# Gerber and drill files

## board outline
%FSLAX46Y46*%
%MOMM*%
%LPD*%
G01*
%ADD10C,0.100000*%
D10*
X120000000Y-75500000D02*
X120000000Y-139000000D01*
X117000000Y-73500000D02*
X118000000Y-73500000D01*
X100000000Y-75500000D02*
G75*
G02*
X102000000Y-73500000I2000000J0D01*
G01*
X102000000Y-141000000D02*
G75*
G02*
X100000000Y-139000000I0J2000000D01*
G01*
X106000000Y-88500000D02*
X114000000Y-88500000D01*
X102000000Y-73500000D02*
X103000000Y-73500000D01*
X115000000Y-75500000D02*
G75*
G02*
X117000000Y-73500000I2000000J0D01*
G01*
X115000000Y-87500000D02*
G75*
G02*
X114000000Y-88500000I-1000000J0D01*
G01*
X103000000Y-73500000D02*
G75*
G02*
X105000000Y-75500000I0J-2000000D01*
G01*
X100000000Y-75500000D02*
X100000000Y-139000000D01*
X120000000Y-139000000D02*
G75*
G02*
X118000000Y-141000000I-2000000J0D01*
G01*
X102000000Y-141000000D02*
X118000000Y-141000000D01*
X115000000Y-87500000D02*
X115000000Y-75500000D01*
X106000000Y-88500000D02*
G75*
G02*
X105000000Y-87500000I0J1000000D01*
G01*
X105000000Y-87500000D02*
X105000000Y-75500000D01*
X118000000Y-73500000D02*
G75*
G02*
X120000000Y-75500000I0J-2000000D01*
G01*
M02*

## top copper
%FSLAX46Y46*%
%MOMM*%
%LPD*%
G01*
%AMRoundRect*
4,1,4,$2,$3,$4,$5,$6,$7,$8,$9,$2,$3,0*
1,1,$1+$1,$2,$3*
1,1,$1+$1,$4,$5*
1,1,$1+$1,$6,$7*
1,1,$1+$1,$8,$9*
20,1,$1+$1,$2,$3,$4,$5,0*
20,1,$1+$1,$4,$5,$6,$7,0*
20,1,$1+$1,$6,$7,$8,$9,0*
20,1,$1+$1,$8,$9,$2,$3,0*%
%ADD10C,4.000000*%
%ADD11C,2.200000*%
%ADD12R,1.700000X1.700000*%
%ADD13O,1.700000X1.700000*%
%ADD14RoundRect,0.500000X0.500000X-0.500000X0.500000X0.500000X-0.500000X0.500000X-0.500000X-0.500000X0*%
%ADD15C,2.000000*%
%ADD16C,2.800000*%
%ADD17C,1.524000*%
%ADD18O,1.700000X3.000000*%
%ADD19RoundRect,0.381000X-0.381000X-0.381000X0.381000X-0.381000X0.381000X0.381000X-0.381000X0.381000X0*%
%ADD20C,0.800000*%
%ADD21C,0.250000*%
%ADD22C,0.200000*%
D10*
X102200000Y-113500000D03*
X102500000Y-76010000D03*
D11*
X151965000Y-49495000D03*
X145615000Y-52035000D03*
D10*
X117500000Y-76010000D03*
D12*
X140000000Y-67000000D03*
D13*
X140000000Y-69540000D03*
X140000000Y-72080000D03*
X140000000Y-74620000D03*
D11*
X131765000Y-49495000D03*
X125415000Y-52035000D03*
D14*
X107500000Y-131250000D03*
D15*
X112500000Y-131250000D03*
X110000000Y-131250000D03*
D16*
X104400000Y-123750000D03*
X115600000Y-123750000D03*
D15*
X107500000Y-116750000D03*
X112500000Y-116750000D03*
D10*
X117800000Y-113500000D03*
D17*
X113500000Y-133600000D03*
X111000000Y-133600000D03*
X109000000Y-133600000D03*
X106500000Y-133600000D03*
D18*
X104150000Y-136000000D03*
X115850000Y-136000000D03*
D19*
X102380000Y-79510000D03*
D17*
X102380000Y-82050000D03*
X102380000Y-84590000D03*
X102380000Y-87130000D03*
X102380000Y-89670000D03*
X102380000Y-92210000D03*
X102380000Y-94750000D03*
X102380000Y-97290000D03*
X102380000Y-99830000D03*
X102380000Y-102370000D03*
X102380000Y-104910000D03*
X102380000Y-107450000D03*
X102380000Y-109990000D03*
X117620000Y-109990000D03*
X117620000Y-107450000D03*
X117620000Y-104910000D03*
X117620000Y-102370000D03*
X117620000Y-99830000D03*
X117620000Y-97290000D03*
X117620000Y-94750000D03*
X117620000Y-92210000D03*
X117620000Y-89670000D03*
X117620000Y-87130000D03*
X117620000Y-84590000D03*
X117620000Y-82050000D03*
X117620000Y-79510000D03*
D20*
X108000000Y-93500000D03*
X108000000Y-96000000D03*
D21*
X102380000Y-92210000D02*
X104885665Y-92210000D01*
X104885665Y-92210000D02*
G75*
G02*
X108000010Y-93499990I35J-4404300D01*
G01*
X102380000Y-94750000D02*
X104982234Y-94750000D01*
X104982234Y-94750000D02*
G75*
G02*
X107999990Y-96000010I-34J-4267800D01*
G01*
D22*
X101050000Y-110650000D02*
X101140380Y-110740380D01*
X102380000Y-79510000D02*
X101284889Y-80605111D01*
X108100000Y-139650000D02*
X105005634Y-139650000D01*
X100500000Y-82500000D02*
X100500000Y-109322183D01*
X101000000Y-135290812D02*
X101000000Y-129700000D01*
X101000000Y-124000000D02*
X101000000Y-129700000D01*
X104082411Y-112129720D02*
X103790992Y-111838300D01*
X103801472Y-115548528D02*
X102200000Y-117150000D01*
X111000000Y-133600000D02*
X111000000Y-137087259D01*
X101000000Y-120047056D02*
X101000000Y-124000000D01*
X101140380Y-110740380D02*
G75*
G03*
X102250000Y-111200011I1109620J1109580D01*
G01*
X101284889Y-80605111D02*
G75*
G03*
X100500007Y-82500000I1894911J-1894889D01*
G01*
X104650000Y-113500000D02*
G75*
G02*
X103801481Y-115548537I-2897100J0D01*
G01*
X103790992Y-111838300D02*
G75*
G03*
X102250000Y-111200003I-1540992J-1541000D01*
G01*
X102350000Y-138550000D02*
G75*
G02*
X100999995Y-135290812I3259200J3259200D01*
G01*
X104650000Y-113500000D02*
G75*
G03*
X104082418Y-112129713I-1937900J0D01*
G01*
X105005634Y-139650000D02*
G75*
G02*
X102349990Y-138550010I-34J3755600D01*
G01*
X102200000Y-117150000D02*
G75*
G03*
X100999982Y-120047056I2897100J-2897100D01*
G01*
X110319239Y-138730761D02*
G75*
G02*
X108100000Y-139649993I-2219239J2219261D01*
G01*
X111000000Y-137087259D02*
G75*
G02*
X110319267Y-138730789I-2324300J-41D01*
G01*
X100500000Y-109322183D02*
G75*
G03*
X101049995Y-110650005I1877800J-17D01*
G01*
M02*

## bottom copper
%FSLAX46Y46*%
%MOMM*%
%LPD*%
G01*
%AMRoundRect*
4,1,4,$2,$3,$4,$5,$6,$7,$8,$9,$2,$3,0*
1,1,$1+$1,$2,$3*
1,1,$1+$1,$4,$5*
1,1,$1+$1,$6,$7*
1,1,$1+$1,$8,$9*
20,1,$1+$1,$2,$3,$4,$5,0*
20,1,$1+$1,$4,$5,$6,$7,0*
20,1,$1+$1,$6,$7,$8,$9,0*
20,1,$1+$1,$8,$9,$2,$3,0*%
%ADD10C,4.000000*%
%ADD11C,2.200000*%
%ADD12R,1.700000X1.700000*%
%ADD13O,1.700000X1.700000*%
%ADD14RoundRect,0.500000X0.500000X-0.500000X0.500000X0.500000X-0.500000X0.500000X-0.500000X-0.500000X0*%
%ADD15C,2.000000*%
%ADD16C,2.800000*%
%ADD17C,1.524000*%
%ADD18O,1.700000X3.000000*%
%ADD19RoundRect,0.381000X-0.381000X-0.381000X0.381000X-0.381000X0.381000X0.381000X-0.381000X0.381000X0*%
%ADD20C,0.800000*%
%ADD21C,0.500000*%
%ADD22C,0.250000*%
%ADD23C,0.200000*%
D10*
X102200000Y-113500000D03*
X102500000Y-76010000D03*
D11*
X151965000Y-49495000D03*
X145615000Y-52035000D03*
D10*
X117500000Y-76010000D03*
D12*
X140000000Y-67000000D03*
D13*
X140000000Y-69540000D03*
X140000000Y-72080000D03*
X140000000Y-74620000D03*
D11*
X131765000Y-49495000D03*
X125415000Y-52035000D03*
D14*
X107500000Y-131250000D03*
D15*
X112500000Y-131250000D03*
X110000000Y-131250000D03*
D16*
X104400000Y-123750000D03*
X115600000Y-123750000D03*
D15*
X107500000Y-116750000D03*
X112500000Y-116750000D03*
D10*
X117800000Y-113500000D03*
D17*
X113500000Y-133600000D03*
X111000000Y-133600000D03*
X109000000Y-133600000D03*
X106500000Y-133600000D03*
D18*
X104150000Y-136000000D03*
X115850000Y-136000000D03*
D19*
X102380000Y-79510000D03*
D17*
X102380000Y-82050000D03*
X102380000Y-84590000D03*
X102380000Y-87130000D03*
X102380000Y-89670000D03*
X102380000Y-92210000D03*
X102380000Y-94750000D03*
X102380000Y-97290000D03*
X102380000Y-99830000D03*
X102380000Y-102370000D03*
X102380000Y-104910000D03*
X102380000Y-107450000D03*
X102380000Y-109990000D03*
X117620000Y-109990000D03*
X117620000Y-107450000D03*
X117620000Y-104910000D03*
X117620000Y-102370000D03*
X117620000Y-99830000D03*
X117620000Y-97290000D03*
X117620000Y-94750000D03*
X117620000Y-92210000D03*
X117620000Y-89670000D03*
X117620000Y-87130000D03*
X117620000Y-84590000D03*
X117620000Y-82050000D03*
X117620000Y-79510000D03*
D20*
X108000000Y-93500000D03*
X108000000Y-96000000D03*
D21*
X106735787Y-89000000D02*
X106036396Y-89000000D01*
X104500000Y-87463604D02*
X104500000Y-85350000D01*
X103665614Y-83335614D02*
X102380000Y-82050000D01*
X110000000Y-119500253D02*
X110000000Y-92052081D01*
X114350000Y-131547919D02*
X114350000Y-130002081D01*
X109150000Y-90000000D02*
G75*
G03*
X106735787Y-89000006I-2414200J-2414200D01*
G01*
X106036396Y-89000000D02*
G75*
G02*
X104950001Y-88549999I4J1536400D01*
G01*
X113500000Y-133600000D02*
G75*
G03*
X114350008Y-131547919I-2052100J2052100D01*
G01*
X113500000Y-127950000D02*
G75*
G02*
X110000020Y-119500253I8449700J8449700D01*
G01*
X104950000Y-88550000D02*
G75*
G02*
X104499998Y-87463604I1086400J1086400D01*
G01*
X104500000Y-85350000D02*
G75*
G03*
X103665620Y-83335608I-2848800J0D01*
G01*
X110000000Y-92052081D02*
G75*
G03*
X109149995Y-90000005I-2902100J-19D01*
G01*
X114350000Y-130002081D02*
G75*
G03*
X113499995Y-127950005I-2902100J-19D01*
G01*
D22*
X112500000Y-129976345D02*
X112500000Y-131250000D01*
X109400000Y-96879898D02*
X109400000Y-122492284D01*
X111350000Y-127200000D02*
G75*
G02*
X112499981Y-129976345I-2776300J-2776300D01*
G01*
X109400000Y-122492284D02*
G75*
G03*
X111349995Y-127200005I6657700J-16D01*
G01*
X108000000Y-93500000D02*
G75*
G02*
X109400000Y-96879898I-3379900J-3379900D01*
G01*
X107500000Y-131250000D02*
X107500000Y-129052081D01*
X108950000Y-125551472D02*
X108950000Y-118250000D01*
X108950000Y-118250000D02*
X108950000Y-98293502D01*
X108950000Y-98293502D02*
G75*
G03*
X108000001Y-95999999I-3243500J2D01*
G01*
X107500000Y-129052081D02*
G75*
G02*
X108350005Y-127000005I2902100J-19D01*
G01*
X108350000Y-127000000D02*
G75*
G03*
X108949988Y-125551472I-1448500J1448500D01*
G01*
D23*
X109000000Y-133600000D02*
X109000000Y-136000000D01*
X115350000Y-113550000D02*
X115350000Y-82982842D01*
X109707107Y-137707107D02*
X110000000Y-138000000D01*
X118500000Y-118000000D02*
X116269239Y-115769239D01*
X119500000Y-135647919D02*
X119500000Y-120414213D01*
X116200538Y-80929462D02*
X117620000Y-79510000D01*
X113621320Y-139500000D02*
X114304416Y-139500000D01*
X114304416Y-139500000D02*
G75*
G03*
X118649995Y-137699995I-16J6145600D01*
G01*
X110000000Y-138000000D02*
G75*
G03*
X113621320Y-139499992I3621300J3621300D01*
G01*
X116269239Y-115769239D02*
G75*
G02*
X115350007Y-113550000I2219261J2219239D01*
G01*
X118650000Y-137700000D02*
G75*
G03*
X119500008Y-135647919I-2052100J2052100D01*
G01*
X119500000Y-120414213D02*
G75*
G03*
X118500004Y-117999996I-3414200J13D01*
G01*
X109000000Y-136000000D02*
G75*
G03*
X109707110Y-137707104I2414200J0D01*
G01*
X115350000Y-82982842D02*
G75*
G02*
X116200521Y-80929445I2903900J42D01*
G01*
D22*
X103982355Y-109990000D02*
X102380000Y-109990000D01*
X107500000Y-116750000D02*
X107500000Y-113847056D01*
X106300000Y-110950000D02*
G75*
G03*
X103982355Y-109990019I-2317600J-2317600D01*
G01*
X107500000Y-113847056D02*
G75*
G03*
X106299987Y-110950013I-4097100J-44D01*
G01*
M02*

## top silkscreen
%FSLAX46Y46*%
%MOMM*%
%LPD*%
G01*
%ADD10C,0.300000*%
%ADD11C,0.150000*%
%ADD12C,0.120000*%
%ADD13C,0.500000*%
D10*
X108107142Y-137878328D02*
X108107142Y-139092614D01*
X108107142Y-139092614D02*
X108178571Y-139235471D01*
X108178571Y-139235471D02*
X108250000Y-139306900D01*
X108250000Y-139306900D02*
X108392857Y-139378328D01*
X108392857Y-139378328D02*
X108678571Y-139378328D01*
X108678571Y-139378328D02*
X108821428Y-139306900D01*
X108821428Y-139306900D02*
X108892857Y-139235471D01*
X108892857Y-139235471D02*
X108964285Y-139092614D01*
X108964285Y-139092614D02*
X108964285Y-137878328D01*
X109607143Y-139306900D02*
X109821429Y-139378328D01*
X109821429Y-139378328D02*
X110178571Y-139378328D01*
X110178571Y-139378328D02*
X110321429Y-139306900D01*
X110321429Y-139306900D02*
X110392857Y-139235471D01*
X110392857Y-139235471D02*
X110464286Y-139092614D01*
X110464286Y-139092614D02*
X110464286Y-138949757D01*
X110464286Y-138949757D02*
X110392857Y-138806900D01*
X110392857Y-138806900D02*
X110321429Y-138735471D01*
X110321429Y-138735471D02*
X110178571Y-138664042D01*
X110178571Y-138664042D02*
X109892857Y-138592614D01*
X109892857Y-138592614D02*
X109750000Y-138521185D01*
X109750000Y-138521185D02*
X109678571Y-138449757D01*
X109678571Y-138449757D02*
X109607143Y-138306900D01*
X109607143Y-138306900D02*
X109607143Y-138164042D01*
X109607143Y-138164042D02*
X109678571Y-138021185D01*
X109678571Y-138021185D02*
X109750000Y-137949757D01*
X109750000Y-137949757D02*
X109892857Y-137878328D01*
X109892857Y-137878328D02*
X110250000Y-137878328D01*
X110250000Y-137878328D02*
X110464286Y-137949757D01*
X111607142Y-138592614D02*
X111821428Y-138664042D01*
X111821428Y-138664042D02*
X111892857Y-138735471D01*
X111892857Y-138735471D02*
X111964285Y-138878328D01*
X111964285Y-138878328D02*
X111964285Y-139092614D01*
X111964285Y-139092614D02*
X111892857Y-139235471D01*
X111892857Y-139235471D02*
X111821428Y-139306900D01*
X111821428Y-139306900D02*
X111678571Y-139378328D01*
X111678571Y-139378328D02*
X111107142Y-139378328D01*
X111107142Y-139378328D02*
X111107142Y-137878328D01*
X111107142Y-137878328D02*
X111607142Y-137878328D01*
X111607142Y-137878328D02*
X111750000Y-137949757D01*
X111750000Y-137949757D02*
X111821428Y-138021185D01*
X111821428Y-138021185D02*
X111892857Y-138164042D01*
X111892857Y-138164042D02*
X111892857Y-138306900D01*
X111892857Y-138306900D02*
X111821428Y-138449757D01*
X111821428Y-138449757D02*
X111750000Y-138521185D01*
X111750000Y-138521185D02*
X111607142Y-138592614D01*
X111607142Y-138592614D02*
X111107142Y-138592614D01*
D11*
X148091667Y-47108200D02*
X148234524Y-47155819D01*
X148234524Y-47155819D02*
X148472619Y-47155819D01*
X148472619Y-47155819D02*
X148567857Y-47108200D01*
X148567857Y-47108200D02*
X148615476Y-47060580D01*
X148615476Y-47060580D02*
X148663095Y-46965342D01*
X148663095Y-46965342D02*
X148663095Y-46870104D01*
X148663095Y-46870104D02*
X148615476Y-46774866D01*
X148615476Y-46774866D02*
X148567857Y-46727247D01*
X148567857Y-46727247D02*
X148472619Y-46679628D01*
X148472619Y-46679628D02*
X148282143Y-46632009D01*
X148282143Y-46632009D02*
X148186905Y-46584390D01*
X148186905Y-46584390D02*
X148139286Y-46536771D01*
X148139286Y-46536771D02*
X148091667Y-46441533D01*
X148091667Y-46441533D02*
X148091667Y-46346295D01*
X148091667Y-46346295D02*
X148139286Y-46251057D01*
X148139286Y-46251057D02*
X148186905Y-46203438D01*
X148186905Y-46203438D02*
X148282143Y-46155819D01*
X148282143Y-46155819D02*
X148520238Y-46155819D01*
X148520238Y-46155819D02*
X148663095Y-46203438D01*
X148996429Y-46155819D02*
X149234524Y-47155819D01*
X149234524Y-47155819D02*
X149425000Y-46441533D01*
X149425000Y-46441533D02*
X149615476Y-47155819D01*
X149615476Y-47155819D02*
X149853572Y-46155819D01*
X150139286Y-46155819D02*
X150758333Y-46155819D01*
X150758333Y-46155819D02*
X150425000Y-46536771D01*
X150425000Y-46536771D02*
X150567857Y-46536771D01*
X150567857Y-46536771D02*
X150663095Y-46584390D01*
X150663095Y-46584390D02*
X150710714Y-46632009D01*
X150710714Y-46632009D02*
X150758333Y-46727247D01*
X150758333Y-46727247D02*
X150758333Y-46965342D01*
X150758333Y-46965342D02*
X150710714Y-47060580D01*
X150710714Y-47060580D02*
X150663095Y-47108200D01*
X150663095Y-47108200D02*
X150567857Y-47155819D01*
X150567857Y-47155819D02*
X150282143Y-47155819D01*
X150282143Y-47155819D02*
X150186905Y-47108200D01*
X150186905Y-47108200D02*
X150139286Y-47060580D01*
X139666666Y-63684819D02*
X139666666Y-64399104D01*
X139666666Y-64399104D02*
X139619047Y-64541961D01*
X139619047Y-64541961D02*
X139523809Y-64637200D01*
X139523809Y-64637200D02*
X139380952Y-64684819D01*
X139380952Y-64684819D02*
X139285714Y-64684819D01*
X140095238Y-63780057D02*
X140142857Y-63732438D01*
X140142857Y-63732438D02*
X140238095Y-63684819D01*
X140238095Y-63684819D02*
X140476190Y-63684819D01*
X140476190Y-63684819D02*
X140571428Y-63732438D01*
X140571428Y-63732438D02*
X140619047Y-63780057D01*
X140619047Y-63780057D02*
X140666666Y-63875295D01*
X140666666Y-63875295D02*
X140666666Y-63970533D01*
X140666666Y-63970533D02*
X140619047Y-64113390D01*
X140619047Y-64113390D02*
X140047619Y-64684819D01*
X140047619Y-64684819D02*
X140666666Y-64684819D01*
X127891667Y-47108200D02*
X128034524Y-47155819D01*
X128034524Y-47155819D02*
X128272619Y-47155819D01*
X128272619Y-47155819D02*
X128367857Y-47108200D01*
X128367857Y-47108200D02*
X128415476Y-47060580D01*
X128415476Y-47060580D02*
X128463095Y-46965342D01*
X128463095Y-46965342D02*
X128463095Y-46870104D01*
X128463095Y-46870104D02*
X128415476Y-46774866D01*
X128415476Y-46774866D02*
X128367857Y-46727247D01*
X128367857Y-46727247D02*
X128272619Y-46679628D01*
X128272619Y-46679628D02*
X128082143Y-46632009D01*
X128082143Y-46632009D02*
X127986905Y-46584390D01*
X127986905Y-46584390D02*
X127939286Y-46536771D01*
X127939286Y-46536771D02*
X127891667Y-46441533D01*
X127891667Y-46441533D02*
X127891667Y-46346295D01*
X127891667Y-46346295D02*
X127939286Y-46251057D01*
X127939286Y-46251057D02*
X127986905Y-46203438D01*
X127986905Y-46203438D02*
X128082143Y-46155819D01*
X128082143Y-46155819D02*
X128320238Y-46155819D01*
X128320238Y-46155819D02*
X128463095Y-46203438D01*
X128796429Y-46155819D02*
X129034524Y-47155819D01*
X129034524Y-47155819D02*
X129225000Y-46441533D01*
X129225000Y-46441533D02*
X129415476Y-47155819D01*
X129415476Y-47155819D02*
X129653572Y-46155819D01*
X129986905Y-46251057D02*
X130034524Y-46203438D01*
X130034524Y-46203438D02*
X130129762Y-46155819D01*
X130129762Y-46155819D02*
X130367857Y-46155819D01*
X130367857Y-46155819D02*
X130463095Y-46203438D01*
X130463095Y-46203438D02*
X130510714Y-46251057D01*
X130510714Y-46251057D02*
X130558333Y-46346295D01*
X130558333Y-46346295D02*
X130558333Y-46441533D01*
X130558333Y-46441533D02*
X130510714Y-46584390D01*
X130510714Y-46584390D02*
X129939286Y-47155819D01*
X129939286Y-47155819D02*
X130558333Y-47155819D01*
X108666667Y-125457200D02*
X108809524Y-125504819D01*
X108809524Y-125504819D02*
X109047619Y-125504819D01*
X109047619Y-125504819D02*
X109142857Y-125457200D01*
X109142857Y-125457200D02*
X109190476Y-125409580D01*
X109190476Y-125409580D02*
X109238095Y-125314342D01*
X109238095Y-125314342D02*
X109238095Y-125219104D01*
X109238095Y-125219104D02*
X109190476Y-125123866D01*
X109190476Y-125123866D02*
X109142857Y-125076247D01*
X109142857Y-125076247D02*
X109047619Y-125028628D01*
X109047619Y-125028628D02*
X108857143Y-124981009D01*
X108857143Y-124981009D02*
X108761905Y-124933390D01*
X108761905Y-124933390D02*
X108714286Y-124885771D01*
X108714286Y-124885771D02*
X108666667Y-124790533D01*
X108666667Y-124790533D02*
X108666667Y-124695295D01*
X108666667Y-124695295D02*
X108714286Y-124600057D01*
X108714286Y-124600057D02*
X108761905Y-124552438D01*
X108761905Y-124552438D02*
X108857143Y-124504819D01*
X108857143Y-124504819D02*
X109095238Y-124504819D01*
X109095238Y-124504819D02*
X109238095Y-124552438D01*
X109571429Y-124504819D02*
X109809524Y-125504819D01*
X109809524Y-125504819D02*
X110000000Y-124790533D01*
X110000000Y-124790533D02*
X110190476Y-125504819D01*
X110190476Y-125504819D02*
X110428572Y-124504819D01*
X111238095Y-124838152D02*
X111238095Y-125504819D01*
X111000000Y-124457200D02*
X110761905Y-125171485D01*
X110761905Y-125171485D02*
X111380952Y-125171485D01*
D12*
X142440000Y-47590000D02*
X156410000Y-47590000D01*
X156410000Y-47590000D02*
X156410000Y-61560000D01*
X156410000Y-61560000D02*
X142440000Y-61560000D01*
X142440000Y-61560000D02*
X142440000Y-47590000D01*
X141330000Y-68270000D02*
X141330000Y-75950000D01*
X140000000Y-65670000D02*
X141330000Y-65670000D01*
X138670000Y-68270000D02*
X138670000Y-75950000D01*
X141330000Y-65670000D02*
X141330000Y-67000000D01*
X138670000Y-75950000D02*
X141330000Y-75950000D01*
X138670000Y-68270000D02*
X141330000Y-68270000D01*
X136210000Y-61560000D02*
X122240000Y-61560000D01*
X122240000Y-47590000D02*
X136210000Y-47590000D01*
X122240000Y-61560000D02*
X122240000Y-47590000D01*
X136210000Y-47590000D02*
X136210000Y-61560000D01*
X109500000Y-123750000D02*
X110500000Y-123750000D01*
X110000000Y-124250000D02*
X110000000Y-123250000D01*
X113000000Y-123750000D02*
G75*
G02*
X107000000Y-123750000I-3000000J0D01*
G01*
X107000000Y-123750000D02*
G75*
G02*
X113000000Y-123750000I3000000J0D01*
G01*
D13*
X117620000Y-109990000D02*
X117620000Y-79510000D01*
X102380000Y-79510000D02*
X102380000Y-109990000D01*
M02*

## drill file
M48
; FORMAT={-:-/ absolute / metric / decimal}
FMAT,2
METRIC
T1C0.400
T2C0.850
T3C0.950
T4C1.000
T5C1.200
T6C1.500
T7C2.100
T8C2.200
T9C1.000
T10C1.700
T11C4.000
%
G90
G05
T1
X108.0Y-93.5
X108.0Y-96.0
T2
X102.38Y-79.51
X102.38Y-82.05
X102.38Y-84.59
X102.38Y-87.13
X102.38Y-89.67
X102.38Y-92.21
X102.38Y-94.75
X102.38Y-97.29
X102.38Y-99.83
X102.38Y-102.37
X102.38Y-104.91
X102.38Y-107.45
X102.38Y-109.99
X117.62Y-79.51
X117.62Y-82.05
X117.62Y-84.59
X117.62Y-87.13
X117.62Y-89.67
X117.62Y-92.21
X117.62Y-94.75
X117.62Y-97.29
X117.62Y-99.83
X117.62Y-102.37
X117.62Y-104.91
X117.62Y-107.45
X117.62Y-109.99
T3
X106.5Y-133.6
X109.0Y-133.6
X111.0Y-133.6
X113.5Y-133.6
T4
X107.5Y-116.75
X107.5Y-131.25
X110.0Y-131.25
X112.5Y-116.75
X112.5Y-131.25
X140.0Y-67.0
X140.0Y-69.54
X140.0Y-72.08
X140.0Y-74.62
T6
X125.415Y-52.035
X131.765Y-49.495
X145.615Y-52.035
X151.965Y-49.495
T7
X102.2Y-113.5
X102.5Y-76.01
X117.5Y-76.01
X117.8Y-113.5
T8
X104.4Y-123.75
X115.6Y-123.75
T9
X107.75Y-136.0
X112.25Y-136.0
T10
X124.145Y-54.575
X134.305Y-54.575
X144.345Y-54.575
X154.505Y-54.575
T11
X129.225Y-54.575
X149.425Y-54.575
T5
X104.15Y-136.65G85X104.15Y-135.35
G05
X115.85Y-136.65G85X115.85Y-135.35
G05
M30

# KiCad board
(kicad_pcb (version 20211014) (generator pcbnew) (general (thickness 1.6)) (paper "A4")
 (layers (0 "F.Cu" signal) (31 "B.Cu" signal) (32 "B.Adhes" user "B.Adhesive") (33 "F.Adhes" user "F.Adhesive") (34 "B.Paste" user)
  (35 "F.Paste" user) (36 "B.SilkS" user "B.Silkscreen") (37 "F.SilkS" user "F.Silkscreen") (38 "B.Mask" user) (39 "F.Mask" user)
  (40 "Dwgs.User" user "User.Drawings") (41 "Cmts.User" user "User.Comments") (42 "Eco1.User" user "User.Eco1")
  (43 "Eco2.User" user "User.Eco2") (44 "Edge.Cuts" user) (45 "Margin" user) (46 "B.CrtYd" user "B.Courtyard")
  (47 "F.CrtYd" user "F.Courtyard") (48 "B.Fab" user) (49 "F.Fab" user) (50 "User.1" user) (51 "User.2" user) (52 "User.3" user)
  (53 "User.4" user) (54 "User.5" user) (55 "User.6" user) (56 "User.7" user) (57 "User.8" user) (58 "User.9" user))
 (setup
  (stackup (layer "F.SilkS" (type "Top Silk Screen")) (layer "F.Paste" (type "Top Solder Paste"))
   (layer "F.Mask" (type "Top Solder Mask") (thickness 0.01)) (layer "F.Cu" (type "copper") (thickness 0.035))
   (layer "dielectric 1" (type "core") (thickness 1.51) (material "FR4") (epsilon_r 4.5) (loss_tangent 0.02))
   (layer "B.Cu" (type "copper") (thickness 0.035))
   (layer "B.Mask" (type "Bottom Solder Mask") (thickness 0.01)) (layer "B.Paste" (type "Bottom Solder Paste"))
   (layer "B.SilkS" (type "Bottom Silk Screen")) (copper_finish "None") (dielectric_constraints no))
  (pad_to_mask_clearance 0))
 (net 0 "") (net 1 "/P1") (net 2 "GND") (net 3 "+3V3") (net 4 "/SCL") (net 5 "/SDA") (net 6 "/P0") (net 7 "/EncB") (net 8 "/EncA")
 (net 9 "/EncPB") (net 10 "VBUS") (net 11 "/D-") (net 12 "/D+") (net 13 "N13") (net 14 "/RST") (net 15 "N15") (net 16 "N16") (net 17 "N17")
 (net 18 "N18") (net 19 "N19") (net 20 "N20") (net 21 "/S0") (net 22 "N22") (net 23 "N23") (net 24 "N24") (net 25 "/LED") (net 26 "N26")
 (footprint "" (layer "F.Cu") (at 102.2 113.5)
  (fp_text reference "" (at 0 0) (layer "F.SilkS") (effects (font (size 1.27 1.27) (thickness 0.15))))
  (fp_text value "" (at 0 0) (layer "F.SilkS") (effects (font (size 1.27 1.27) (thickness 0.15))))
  (pad "103" thru_hole circle (at 0 0) (size 4 4) (drill 2.1) (layers *.Cu *.Mask)))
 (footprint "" (layer "F.Cu") (at 103.6 74.6)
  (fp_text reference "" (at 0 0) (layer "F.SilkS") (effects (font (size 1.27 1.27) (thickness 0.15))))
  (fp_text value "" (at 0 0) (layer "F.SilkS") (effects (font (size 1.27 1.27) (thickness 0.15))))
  (pad "101" thru_hole circle (at -1.1 1.41) (size 4 4) (drill 2.1) (layers *.Cu *.Mask)))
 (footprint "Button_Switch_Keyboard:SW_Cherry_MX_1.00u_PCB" (layer "F.Cu") (at 151.965 49.495)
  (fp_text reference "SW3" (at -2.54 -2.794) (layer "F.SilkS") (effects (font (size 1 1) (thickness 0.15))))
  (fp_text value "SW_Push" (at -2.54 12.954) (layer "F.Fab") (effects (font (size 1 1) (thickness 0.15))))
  (fp_line (start -9.525 -1.905) (end 4.445 -1.905) (layer "F.SilkS") (width 0.12))
  (fp_line (start 4.445 -1.905) (end 4.445 12.065) (layer "F.SilkS") (width 0.12))
  (fp_line (start 4.445 12.065) (end -9.525 12.065) (layer "F.SilkS") (width 0.12))
  (fp_line (start -9.525 12.065) (end -9.525 -1.905) (layer "F.SilkS") (width 0.12))
  (pad "" np_thru_hole circle (at -7.62 5.08) (size 1.7 1.7) (drill 1.7) (layers *.Cu *.Mask))
  (pad "" np_thru_hole circle (at -2.54 5.08) (size 4 4) (drill 4) (layers *.Cu *.Mask))
  (pad "" np_thru_hole circle (at 2.54 5.08) (size 1.7 1.7) (drill 1.7) (layers *.Cu *.Mask))
  (pad "1" thru_hole circle (at 0 0) (size 2.2 2.2) (drill 1.5) (layers *.Cu *.Mask) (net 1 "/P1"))
  (pad "2" thru_hole circle (at -6.35 2.54) (size 2.2 2.2) (drill 1.5) (layers *.Cu *.Mask) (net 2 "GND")))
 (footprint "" (layer "F.Cu") (at 117.5 79)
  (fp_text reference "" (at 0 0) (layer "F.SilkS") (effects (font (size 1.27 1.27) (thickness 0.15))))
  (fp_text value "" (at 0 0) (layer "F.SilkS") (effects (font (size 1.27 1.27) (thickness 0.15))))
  (pad "102" thru_hole circle (at 0 -2.99) (size 4 4) (drill 2.1) (layers *.Cu *.Mask)))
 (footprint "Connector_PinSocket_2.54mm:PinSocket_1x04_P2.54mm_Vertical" (layer "F.Cu") (at 140 67)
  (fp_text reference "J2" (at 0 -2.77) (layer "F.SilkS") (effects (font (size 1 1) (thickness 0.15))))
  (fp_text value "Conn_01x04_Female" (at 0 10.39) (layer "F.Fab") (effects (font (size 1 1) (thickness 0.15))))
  (fp_line (start 1.33 1.27) (end 1.33 8.95) (layer "F.SilkS") (width 0.12))
  (fp_line (start 0 -1.33) (end 1.33 -1.33) (layer "F.SilkS") (width 0.12))
  (fp_line (start -1.33 1.27) (end -1.33 8.95) (layer "F.SilkS") (width 0.12))
  (fp_line (start 1.33 -1.33) (end 1.33 0) (layer "F.SilkS") (width 0.12))
  (fp_line (start -1.33 8.95) (end 1.33 8.95) (layer "F.SilkS") (width 0.12))
  (fp_line (start -1.33 1.27) (end 1.33 1.27) (layer "F.SilkS") (width 0.12))
  (pad "1" thru_hole rect (at 0 0) (size 1.7 1.7) (drill 1) (layers *.Cu *.Mask) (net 2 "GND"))
  (pad "2" thru_hole oval (at 0 2.54) (size 1.7 1.7) (drill 1) (layers *.Cu *.Mask) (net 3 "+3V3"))
  (pad "3" thru_hole oval (at 0 5.08) (size 1.7 1.7) (drill 1) (layers *.Cu *.Mask) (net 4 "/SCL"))
  (pad "4" thru_hole oval (at 0 7.62) (size 1.7 1.7) (drill 1) (layers *.Cu *.Mask) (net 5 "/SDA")))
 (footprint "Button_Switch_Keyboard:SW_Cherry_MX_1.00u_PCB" (layer "F.Cu") (at 131.765 49.495)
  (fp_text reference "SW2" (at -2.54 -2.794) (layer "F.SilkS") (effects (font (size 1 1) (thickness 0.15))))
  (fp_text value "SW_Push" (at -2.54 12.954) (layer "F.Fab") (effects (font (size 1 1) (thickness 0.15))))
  (fp_line (start 4.445 12.065) (end -9.525 12.065) (layer "F.SilkS") (width 0.12))
  (fp_line (start -9.525 -1.905) (end 4.445 -1.905) (layer "F.SilkS") (width 0.12))
  (fp_line (start -9.525 12.065) (end -9.525 -1.905) (layer "F.SilkS") (width 0.12))
  (fp_line (start 4.445 -1.905) (end 4.445 12.065) (layer "F.SilkS") (width 0.12))
  (pad "" np_thru_hole circle (at -2.54 5.08) (size 4 4) (drill 4) (layers *.Cu *.Mask))
  (pad "" np_thru_hole circle (at -7.62 5.08) (size 1.7 1.7) (drill 1.7) (layers *.Cu *.Mask))
  (pad "" np_thru_hole circle (at 2.54 5.08) (size 1.7 1.7) (drill 1.7) (layers *.Cu *.Mask))
  (pad "1" thru_hole circle (at 0 0) (size 2.2 2.2) (drill 1.5) (layers *.Cu *.Mask) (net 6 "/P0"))
  (pad "2" thru_hole circle (at -6.35 2.54) (size 2.2 2.2) (drill 1.5) (layers *.Cu *.Mask) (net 2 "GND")))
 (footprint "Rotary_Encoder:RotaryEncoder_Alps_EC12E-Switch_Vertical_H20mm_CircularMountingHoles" (layer "F.Cu") (at 107.5 131.25 90)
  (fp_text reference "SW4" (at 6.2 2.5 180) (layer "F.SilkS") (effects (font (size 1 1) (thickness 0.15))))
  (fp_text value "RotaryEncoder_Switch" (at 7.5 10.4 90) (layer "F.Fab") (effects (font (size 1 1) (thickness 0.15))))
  (fp_line (start 7.5 2) (end 7.5 3) (layer "F.SilkS") (width 0.12))
  (fp_line (start 7 2.5) (end 8 2.5) (layer "F.SilkS") (width 0.12))
  (fp_circle (center 7.5 2.5) (end 10.5 2.5) (layer "F.SilkS") (width 0.12) (fill none))
  (pad "A" thru_hole roundrect (at 0 0 90) (size 2 2) (drill 1) (layers *.Cu *.Mask) (roundrect_rratio 0.25) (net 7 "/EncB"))
  (pad "B" thru_hole circle (at 0 5 90) (size 2 2) (drill 1) (layers *.Cu *.Mask) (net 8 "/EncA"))
  (pad "C" thru_hole circle (at 0 2.5 90) (size 2 2) (drill 1) (layers *.Cu *.Mask) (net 2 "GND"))
  (pad "MP" thru_hole circle (at 7.5 -3.1 90) (size 2.8 2.8) (drill 2.2) (layers *.Cu *.Mask))
  (pad "MP" thru_hole circle (at 7.5 8.1 90) (size 2.8 2.8) (drill 2.2) (layers *.Cu *.Mask))
  (pad "S1" thru_hole circle (at 14.5 0 90) (size 2 2) (drill 1) (layers *.Cu *.Mask) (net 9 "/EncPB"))
  (pad "S2" thru_hole circle (at 14.5 5 90) (size 2 2) (drill 1) (layers *.Cu *.Mask) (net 2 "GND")))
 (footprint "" (layer "F.Cu") (at 117.8 112)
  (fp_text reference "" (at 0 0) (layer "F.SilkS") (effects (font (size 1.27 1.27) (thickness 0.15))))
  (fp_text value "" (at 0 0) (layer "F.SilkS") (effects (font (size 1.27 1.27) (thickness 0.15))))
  (pad "104" thru_hole circle (at 0 1.5) (size 4 4) (drill 2.1) (layers *.Cu *.Mask)))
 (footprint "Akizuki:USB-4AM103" (layer "F.Cu") (at 110 135 180)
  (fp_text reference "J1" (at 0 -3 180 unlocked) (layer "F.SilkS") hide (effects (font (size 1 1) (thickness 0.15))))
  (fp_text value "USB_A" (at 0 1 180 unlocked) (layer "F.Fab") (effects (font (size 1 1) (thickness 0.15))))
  (pad "" np_thru_hole circle (at 2.25 -1 180) (size 1 1) (drill 1) (layers *.Mask))
  (pad "" np_thru_hole circle (at -2.25 -1 180) (size 1 1) (drill 1) (layers *.Mask))
  (pad "1" thru_hole circle (at -3.5 1.4 180) (size 1.524 1.524) (drill 0.95) (layers *.Cu *.Mask) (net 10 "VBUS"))
  (pad "2" thru_hole circle (at -1 1.4 180) (size 1.524 1.524) (drill 0.95) (layers *.Cu *.Mask) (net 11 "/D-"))
  (pad "3" thru_hole circle (at 1 1.4 180) (size 1.524 1.524) (drill 0.95) (layers *.Cu *.Mask) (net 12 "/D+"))
  (pad "4" thru_hole circle (at 3.5 1.4 180) (size 1.524 1.524) (drill 0.95) (layers *.Cu *.Mask) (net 2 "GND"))
  (pad "5" thru_hole oval (at 5.85 -1 180) (size 1.7 3) (drill oval 1.2 2.5) (layers *.Cu *.Mask) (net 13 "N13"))
  (pad "5" thru_hole oval (at -5.85 -1 180) (size 1.7 3) (drill oval 1.2 2.5) (layers *.Cu *.Mask) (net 13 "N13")))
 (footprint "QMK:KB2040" (layer "F.Cu") (at 110 94.75)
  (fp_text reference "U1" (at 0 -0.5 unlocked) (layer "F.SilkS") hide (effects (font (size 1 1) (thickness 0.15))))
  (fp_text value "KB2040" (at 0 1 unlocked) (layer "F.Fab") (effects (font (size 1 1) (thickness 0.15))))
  (fp_line (start 7.62 15.24) (end 7.62 -15.24) (layer "F.SilkS") (width 0.5))
  (fp_line (start -7.62 -15.24) (end -7.62 15.24) (layer "F.SilkS") (width 0.5))
  (pad "0" thru_hole roundrect (at -7.62 -15.24) (size 1.524 1.524) (drill 0.85) (layers *.Cu *.Mask) (roundrect_rratio 0.25) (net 11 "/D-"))
  (pad "1" thru_hole circle (at -7.62 -12.7) (size 1.524 1.524) (drill 0.85) (layers *.Cu *.Mask) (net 10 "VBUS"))
  (pad "2" thru_hole circle (at -7.62 -10.16) (size 1.524 1.524) (drill 0.85) (layers *.Cu *.Mask) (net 2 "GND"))
  (pad "3" thru_hole circle (at -7.62 -7.62) (size 1.524 1.524) (drill 0.85) (layers *.Cu *.Mask) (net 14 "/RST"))
  (pad "4" thru_hole circle (at -7.62 -5.08) (size 1.524 1.524) (drill 0.85) (layers *.Cu *.Mask) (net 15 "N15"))
  (pad "5" thru_hole circle (at -7.62 -2.54) (size 1.524 1.524) (drill 0.85) (layers *.Cu *.Mask) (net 8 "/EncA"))
  (pad "6" thru_hole circle (at -7.62 0) (size 1.524 1.524) (drill 0.85) (layers *.Cu *.Mask) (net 7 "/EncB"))
  (pad "7" thru_hole circle (at -7.62 2.54) (size 1.524 1.524) (drill 0.85) (layers *.Cu *.Mask) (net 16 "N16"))
  (pad "8" thru_hole circle (at -7.62 5.08) (size 1.524 1.524) (drill 0.85) (layers *.Cu *.Mask) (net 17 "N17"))
  (pad "9" thru_hole circle (at -7.62 7.62) (size 1.524 1.524) (drill 0.85) (layers *.Cu *.Mask) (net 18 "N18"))
  (pad "10" thru_hole circle (at -7.62 10.16) (size 1.524 1.524) (drill 0.85) (layers *.Cu *.Mask) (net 6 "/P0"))
  (pad "11" thru_hole circle (at -7.62 12.7) (size 1.524 1.524) (drill 0.85) (layers *.Cu *.Mask) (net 1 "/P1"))
  (pad "12" thru_hole circle (at -7.62 15.24) (size 1.524 1.524) (drill 0.85) (layers *.Cu *.Mask) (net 9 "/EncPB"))
  (pad "13" thru_hole circle (at 7.62 15.24) (size 1.524 1.524) (drill 0.85) (layers *.Cu *.Mask) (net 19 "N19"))
  (pad "14" thru_hole circle (at 7.62 12.7) (size 1.524 1.524) (drill 0.85) (layers *.Cu *.Mask) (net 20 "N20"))
  (pad "15" thru_hole circle (at 7.62 10.16) (size 1.524 1.524) (drill 0.85) (layers *.Cu *.Mask) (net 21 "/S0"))
  (pad "16" thru_hole circle (at 7.62 7.62) (size 1.524 1.524) (drill 0.85) (layers *.Cu *.Mask) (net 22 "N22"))
  (pad "17" thru_hole circle (at 7.62 5.08) (size 1.524 1.524) (drill 0.85) (layers *.Cu *.Mask) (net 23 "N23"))
  (pad "18" thru_hole circle (at 7.62 2.54) (size 1.524 1.524) (drill 0.85) (layers *.Cu *.Mask) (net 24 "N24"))
  (pad "19" thru_hole circle (at 7.62 0) (size 1.524 1.524) (drill 0.85) (layers *.Cu *.Mask) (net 4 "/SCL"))
  (pad "20" thru_hole circle (at 7.62 -2.54) (size 1.524 1.524) (drill 0.85) (layers *.Cu *.Mask) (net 5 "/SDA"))
  (pad "21" thru_hole circle (at 7.62 -5.08) (size 1.524 1.524) (drill 0.85) (layers *.Cu *.Mask) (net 2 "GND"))
  (pad "22" thru_hole circle (at 7.62 -7.62) (size 1.524 1.524) (drill 0.85) (layers *.Cu *.Mask) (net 2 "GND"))
  (pad "23" thru_hole circle (at 7.62 -10.16) (size 1.524 1.524) (drill 0.85) (layers *.Cu *.Mask) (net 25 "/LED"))
  (pad "24" thru_hole circle (at 7.62 -12.7) (size 1.524 1.524) (drill 0.85) (layers *.Cu *.Mask) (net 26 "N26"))
  (pad "25" thru_hole circle (at 7.62 -15.24) (size 1.524 1.524) (drill 0.85) (layers *.Cu *.Mask) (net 12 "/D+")))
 (gr_line (start 120 75.5) (end 120 139) (layer "Edge.Cuts") (width 0.1))
 (gr_line (start 117 73.5) (end 118 73.5) (layer "Edge.Cuts") (width 0.1))
 (gr_arc (start 100 75.5) (mid 100.585786 74.085786) (end 102 73.5) (layer "Edge.Cuts") (width 0.1))
 (gr_arc (start 102 141) (mid 100.585786 140.414214) (end 100 139) (layer "Edge.Cuts") (width 0.1))
 (gr_line (start 106 88.5) (end 114 88.5) (layer "Edge.Cuts") (width 0.1))
 (gr_line (start 102 73.5) (end 103 73.5) (layer "Edge.Cuts") (width 0.1))
 (gr_arc (start 115 75.5) (mid 115.585786 74.085786) (end 117 73.5) (layer "Edge.Cuts") (width 0.1))
 (gr_arc (start 115 87.5) (mid 114.707107 88.207107) (end 114 88.5) (layer "Edge.Cuts") (width 0.1))
 (gr_arc (start 103 73.5) (mid 104.414214 74.085786) (end 105 75.5) (layer "Edge.Cuts") (width 0.1))
 (gr_line (start 100 75.5) (end 100 139) (layer "Edge.Cuts") (width 0.1))
 (gr_arc (start 120 139) (mid 119.414214 140.414214) (end 118 141) (layer "Edge.Cuts") (width 0.1))
 (gr_line (start 102 141) (end 118 141) (layer "Edge.Cuts") (width 0.1))
 (gr_line (start 115 87.5) (end 115 75.5) (layer "Edge.Cuts") (width 0.1))
 (gr_arc (start 106 88.5) (mid 105.292893 88.207107) (end 105 87.5) (layer "Edge.Cuts") (width 0.1))
 (gr_line (start 105 87.5) (end 105 75.5) (layer "Edge.Cuts") (width 0.1))
 (gr_arc (start 118 73.5) (mid 119.414214 74.085786) (end 120 75.5) (layer "Edge.Cuts") (width 0.1))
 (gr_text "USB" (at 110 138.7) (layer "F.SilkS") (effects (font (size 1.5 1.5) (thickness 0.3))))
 (segment (start 106.735787 89) (end 106.036396 89) (width 0.5) (layer "B.Cu") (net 10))
 (segment (start 104.5 87.463604) (end 104.5 85.35) (width 0.5) (layer "B.Cu") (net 10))
 (segment (start 103.665614 83.335614) (end 102.38 82.05) (width 0.5) (layer "B.Cu") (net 10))
 (segment (start 110 119.500253) (end 110 92.052081) (width 0.5) (layer "B.Cu") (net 10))
 (segment (start 114.35 131.547919) (end 114.35 130.002081) (width 0.5) (layer "B.Cu") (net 10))
 (arc (start 109.15 90) (mid 108.04235 89.259891) (end 106.735787 89) (width 0.5) (layer "B.Cu") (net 10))
 (arc (start 106.036396 89) (mid 105.448443 88.883049) (end 104.95 88.55) (width 0.5) (layer "B.Cu") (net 10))
 (arc (start 113.5 133.6) (mid 114.129092 132.658497) (end 114.35 131.547919) (width 0.5) (layer "B.Cu") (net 10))
 (arc (start 113.5 127.95) (mid 110.90962 124.073223) (end 110 119.500253) (width 0.5) (layer "B.Cu") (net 10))
 (arc (start 104.95 88.55) (mid 104.616951 88.051558) (end 104.5 87.463604) (width 0.5) (layer "B.Cu") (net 10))
 (arc (start 104.5 85.35) (mid 104.28315 84.259822) (end 103.665614 83.335614) (width 0.5) (layer "B.Cu") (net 10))
 (arc (start 110 92.052081) (mid 109.779092 90.941503) (end 109.15 90) (width 0.5) (layer "B.Cu") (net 10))
 (arc (start 114.35 130.002081) (mid 114.129092 128.891503) (end 113.5 127.95) (width 0.5) (layer "B.Cu") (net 10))
 (segment (start 102.38 92.21) (end 104.885665 92.21) (width 0.25) (layer "F.Cu") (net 8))
 (via (at 108 93.5) (size 0.8) (drill 0.4) (layers "F.Cu" "B.Cu") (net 8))
 (arc (start 104.885665 92.21) (mid 106.571131 92.54526) (end 108 93.5) (width 0.25) (layer "F.Cu") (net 8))
 (segment (start 112.5 129.976345) (end 112.5 131.25) (width 0.25) (layer "B.Cu") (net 8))
 (segment (start 109.4 96.879898) (end 109.4 122.492284) (width 0.25) (layer "B.Cu") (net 8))
 (arc (start 111.35 127.2) (mid 112.201125 128.473798) (end 112.5 129.976345) (width 0.25) (layer "B.Cu") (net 8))
 (arc (start 109.4 122.492284) (mid 109.906789 125.040081) (end 111.35 127.2) (width 0.25) (layer "B.Cu") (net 8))
 (arc (start 108 93.5) (mid 109.036152 95.05071) (end 109.4 96.879898) (width 0.25) (layer "B.Cu") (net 8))
 (segment (start 102.38 94.75) (end 104.982234 94.75) (width 0.25) (layer "F.Cu") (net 7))
 (via (at 108 96) (size 0.8) (drill 0.4) (layers "F.Cu" "B.Cu") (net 7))
 (arc (start 104.982234 94.75) (mid 106.615437 95.074865) (end 108 96) (width 0.25) (layer "F.Cu") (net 7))
 (segment (start 107.5 131.25) (end 107.5 129.052081) (width 0.25) (layer "B.Cu") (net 7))
 (segment (start 108.95 125.551472) (end 108.95 118.25) (width 0.25) (layer "B.Cu") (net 7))
 (segment (start 108.95 118.25) (end 108.95 98.293502) (width 0.25) (layer "B.Cu") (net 7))
 (arc (start 108.95 98.293502) (mid 108.703103 97.052268) (end 108 96) (width 0.25) (layer "B.Cu") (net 7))
 (arc (start 107.5 129.052081) (mid 107.720908 127.941503) (end 108.35 127) (width 0.25) (layer "B.Cu") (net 7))
 (arc (start 108.35 127) (mid 108.794065 126.33541) (end 108.95 125.551472) (width 0.25) (layer "B.Cu") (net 7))
 (segment (start 109 133.6) (end 109 136) (width 0.2) (layer "B.Cu") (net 12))
 (segment (start 115.35 113.55) (end 115.35 82.982842) (width 0.2) (layer "B.Cu") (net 12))
 (segment (start 109.707107 137.707107) (end 110 138) (width 0.2) (layer "B.Cu") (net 12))
 (segment (start 118.5 118) (end 116.269239 115.769239) (width 0.2) (layer "B.Cu") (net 12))
 (segment (start 119.5 135.647919) (end 119.5 120.414213) (width 0.2) (layer "B.Cu") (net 12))
 (segment (start 116.200538 80.929462) (end 117.62 79.51) (width 0.2) (layer "B.Cu") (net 12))
 (segment (start 113.62132 139.5) (end 114.304416 139.5) (width 0.2) (layer "B.Cu") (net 12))
 (arc (start 114.304416 139.5) (mid 116.656229 139.032195) (end 118.65 137.7) (width 0.2) (layer "B.Cu") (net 12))
 (arc (start 110 138) (mid 111.661476 139.110163) (end 113.62132 139.5) (width 0.2) (layer "B.Cu") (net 12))
 (arc (start 116.269239 115.769239) (mid 115.588902 114.751044) (end 115.35 113.55) (width 0.2) (layer "B.Cu") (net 12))
 (arc (start 118.65 137.7) (mid 119.279092 136.758497) (end 119.5 135.647919) (width 0.2) (layer "B.Cu") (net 12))
 (arc (start 119.5 120.414213) (mid 119.240108 119.10765) (end 118.5 118) (width 0.2) (layer "B.Cu") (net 12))
 (arc (start 109 136) (mid 109.183771 136.92388) (end 109.707107 137.707107) (width 0.2) (layer "B.Cu") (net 12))
 (arc (start 115.35 82.982842) (mid 115.571048 81.871561) (end 116.200538 80.929462) (width 0.2) (layer "B.Cu") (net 12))
 (segment (start 103.982355 109.99) (end 102.38 109.99) (width 0.25) (layer "B.Cu") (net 9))
 (segment (start 107.5 116.75) (end 107.5 113.847056) (width 0.25) (layer "B.Cu") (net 9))
 (arc (start 106.3 110.95) (mid 105.236656 110.239495) (end 103.982355 109.99) (width 0.25) (layer "B.Cu") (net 9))
 (arc (start 107.5 113.847056) (mid 107.18813 112.279181) (end 106.3 110.95) (width 0.25) (layer "B.Cu") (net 9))
 (segment (start 101.05 110.65) (end 101.14038 110.74038) (width 0.2) (layer "F.Cu") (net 11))
 (segment (start 102.38 79.51) (end 101.284889 80.605111) (width 0.2) (layer "F.Cu") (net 11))
 (segment (start 108.1 139.65) (end 105.005634 139.65) (width 0.2) (layer "F.Cu") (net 11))
 (segment (start 100.5 82.5) (end 100.5 109.322183) (width 0.2) (layer "F.Cu") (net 11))
 (segment (start 101 135.290812) (end 101 129.7) (width 0.2) (layer "F.Cu") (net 11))
 (segment (start 101 124) (end 101 129.7) (width 0.2) (layer "F.Cu") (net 11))
 (segment (start 104.082411 112.12972) (end 103.790992 111.8383) (width 0.2) (layer "F.Cu") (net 11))
 (segment (start 103.801472 115.548528) (end 102.2 117.15) (width 0.2) (layer "F.Cu") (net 11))
 (segment (start 111 133.6) (end 111 137.087259) (width 0.2) (layer "F.Cu") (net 11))
 (segment (start 101 120.047056) (end 101 124) (width 0.2) (layer "F.Cu") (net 11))
 (arc (start 101.14038 110.74038) (mid 101.649478 111.080548) (end 102.25 111.2) (width 0.2) (layer "F.Cu") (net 11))
 (arc (start 101.284889 80.605111) (mid 100.703986 81.474493) (end 100.5 82.5) (width 0.2) (layer "F.Cu") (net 11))
 (arc (start 104.65 113.5) (mid 104.429475 114.608655) (end 103.801472 115.548528) (width 0.2) (layer "F.Cu") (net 11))
 (arc (start 103.790992 111.8383) (mid 103.083979 111.365888) (end 102.25 111.2) (width 0.2) (layer "F.Cu") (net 11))
 (arc (start 102.35 138.55) (mid 101.350854 137.054671) (end 101 135.290812) (width 0.2) (layer "F.Cu") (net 11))
 (arc (start 104.65 113.5) (mid 104.502489 112.75841) (end 104.082411 112.12972) (width 0.2) (layer "F.Cu") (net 11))
 (arc (start 105.005634 139.65) (mid 103.568415 139.364119) (end 102.35 138.55) (width 0.2) (layer "F.Cu") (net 11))
 (arc (start 102.2 117.15) (mid 101.31187 118.47918) (end 101 120.047056) (width 0.2) (layer "F.Cu") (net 11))
 (arc (start 110.319239 138.730761) (mid 109.301044 139.411098) (end 108.1 139.65) (width 0.2) (layer "F.Cu") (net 11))
 (arc (start 111 137.087259) (mid 110.823076 137.976716) (end 110.319239 138.730761) (width 0.2) (layer "F.Cu") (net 11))
 (arc (start 100.5 109.322183) (mid 100.642941 110.040792) (end 101.05 110.65) (width 0.2) (layer "F.Cu") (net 11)))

